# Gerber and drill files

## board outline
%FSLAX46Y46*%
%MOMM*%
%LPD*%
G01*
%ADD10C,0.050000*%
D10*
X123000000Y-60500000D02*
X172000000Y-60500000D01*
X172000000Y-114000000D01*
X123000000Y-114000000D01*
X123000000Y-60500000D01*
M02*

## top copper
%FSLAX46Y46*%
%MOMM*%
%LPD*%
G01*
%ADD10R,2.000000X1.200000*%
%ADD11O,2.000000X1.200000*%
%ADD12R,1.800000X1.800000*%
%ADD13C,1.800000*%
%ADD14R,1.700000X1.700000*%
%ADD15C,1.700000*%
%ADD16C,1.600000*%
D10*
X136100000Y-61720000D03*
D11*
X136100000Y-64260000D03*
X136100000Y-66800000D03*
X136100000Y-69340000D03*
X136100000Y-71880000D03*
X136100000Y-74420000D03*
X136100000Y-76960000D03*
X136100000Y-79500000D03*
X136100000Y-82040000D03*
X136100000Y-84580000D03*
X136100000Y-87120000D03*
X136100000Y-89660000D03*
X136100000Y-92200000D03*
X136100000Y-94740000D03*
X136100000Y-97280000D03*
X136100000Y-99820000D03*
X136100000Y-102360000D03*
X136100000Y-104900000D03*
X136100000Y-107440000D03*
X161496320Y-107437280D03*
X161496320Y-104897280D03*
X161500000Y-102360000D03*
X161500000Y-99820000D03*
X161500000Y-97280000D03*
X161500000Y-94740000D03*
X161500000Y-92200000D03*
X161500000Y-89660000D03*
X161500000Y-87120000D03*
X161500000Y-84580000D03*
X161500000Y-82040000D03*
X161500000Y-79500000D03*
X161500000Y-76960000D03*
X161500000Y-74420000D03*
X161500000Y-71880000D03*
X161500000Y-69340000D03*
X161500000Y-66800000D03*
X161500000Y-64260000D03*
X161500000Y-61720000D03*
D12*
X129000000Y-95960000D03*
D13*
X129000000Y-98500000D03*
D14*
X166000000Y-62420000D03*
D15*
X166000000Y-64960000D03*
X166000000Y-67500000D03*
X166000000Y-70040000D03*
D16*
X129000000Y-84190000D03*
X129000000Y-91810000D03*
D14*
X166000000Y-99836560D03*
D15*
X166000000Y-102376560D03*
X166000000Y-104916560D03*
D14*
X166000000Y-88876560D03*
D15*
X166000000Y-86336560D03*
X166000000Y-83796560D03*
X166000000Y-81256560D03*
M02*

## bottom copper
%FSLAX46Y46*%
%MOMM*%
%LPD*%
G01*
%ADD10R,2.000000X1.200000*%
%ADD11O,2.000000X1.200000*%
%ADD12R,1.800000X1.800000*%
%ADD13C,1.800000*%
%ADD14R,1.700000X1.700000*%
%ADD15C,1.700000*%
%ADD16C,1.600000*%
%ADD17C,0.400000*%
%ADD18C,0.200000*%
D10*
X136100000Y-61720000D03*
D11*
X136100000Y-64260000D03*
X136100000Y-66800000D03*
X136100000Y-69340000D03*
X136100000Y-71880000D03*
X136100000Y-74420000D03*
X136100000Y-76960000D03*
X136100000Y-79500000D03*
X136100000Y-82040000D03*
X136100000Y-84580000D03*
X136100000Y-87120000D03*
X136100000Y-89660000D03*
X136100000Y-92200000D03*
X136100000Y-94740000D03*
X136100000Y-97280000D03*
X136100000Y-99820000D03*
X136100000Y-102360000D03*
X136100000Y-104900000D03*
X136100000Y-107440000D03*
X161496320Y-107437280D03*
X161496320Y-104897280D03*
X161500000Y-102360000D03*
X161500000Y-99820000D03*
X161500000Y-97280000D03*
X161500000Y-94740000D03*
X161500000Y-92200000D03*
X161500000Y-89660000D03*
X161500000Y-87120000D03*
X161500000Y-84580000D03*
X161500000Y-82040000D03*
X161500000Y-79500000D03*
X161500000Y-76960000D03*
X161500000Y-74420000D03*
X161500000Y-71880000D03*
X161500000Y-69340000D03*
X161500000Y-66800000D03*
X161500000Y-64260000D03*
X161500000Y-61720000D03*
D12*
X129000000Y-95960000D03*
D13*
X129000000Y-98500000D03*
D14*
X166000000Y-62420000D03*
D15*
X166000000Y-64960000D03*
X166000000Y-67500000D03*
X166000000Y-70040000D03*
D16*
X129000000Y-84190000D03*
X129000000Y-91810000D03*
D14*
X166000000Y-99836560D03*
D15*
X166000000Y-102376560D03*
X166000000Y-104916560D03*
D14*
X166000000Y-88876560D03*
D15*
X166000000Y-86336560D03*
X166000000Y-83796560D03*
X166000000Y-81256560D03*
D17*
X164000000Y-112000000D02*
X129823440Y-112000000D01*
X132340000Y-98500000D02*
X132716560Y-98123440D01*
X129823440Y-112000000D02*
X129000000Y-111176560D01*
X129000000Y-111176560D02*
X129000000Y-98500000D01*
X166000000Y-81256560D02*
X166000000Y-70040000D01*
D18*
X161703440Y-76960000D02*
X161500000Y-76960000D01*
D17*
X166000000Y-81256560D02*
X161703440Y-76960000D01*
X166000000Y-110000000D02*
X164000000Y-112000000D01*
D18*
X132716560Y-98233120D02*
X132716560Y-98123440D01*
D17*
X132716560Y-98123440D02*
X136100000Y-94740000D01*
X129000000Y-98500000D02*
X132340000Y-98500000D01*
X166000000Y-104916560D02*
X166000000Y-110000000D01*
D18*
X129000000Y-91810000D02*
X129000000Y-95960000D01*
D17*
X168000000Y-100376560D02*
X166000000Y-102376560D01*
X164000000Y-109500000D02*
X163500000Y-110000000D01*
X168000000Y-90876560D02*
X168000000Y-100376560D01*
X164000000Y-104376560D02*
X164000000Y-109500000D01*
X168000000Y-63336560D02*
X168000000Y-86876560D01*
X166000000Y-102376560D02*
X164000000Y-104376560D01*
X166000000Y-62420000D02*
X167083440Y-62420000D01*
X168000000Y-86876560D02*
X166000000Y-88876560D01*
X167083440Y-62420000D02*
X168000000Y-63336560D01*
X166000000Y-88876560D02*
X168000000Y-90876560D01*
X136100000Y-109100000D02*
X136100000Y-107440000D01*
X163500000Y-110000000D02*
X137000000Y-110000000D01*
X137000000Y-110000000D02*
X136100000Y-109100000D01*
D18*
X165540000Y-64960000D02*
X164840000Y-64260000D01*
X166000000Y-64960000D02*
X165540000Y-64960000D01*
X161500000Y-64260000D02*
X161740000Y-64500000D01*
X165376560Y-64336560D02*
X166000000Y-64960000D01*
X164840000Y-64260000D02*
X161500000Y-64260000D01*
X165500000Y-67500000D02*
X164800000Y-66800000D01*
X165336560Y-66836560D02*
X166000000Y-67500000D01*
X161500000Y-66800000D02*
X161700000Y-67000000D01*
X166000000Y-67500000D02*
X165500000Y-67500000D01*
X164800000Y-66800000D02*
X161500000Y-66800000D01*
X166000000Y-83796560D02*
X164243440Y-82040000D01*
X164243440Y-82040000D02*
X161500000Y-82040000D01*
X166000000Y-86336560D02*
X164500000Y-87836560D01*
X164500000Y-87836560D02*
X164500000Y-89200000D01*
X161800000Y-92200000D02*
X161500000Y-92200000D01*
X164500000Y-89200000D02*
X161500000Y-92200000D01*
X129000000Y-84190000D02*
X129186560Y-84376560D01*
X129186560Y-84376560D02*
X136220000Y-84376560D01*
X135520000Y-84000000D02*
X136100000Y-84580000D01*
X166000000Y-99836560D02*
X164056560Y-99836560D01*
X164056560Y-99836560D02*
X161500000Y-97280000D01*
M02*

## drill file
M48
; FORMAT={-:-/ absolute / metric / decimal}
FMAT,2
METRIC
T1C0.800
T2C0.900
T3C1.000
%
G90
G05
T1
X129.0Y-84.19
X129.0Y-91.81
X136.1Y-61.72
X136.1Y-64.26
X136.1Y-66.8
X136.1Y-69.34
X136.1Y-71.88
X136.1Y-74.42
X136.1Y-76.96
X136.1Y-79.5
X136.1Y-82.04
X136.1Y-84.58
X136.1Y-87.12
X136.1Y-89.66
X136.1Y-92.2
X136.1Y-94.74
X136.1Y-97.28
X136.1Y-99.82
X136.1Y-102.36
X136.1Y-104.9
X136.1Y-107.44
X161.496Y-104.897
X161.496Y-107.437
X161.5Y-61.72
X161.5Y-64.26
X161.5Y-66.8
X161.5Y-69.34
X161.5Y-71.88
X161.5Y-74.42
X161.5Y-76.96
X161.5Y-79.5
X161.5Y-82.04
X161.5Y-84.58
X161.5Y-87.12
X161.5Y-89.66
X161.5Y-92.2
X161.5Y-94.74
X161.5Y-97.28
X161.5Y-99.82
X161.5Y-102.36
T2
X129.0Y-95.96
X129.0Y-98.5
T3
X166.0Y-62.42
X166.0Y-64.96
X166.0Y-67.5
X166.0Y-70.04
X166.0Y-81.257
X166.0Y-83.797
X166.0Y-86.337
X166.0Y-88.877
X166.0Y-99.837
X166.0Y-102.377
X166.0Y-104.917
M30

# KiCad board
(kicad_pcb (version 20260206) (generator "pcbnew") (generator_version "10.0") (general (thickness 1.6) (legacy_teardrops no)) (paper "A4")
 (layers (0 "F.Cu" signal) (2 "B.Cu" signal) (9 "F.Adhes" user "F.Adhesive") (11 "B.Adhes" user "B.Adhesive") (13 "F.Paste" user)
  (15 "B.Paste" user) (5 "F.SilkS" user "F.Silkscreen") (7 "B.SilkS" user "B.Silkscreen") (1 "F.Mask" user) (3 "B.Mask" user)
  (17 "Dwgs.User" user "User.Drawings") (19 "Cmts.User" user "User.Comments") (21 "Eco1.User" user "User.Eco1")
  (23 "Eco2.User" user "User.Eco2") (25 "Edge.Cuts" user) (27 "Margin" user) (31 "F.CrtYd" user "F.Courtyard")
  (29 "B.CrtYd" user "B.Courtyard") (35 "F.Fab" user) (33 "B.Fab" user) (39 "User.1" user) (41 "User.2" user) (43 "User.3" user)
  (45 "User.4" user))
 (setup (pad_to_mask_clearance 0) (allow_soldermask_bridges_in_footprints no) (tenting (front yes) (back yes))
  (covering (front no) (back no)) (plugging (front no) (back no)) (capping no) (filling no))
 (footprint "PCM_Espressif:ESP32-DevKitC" (layer "F.Cu") (at 136.1 61.72)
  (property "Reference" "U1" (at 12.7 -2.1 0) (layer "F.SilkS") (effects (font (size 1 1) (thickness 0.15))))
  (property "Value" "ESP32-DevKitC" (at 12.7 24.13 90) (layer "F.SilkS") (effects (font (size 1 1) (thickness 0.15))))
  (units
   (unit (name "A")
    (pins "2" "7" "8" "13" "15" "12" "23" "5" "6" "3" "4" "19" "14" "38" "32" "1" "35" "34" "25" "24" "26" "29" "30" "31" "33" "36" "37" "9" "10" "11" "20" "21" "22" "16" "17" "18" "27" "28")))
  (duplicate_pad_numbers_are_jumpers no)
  (pad "1" thru_hole rect (at 0 0 270) (size 1.2 2) (drill 0.8) (layers "*.Cu" "*.Mask") (remove_unused_layers no)
   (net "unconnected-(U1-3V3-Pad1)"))
  (pad "2" thru_hole oval (at 0 2.54 270) (size 1.2 2) (drill 0.8) (layers "*.Cu" "*.Mask") (remove_unused_layers no)
   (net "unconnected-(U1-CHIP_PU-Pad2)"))
  (pad "3" thru_hole oval (at 0 5.08 270) (size 1.2 2) (drill 0.8) (layers "*.Cu" "*.Mask") (remove_unused_layers no)
   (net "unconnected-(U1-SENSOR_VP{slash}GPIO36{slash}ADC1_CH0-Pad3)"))
  (pad "4" thru_hole oval (at 0 7.62 270) (size 1.2 2) (drill 0.8) (layers "*.Cu" "*.Mask") (remove_unused_layers no)
   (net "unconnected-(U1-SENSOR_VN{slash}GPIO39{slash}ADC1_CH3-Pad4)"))
  (pad "5" thru_hole oval (at 0 10.16 270) (size 1.2 2) (drill 0.8) (layers "*.Cu" "*.Mask") (remove_unused_layers no)
   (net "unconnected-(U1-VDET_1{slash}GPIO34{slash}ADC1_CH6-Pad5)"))
  (pad "6" thru_hole oval (at 0 12.7 270) (size 1.2 2) (drill 0.8) (layers "*.Cu" "*.Mask") (remove_unused_layers no)
   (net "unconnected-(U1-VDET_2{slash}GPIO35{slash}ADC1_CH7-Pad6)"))
  (pad "7" thru_hole oval (at 0 15.24 270) (size 1.2 2) (drill 0.8) (layers "*.Cu" "*.Mask") (remove_unused_layers no)
   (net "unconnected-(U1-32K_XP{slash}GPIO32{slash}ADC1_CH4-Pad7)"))
  (pad "8" thru_hole oval (at 0 17.78 270) (size 1.2 2) (drill 0.8) (layers "*.Cu" "*.Mask") (remove_unused_layers no)
   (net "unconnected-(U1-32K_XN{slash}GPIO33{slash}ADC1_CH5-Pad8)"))
  (pad "9" thru_hole oval (at 0 20.32 270) (size 1.2 2) (drill 0.8) (layers "*.Cu" "*.Mask") (remove_unused_layers no)
   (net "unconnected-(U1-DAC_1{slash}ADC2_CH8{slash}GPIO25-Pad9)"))
  (pad "10" thru_hole oval (at 0 22.86 270) (size 1.2 2) (drill 0.8) (layers "*.Cu" "*.Mask") (remove_unused_layers no)
   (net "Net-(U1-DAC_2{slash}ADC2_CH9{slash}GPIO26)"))
  (pad "11" thru_hole oval (at 0 25.4 270) (size 1.2 2) (drill 0.8) (layers "*.Cu" "*.Mask") (remove_unused_layers no)
   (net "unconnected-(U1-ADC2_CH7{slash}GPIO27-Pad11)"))
  (pad "12" thru_hole oval (at 0 27.94 270) (size 1.2 2) (drill 0.8) (layers "*.Cu" "*.Mask") (remove_unused_layers no)
   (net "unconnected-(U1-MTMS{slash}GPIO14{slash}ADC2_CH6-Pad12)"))
  (pad "13" thru_hole oval (at 0 30.48 270) (size 1.2 2) (drill 0.8) (layers "*.Cu" "*.Mask") (remove_unused_layers no)
   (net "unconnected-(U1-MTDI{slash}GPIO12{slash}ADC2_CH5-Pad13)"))
  (pad "14" thru_hole oval (at 0 33.02 270) (size 1.2 2) (drill 0.8) (layers "*.Cu" "*.Mask") (remove_unused_layers no) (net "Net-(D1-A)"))
  (pad "15" thru_hole oval (at 0 35.56 270) (size 1.2 2) (drill 0.8) (layers "*.Cu" "*.Mask") (remove_unused_layers no)
   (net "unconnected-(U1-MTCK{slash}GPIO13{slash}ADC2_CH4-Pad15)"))
  (pad "16" thru_hole oval (at 0 38.1 270) (size 1.2 2) (drill 0.8) (layers "*.Cu" "*.Mask") (remove_unused_layers no)
   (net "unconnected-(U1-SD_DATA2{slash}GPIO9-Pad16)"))
  (pad "17" thru_hole oval (at 0 40.64 270) (size 1.2 2) (drill 0.8) (layers "*.Cu" "*.Mask") (remove_unused_layers no)
   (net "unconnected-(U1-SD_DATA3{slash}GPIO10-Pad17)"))
  (pad "18" thru_hole oval (at 0 43.18 270) (size 1.2 2) (drill 0.8) (layers "*.Cu" "*.Mask") (remove_unused_layers no)
   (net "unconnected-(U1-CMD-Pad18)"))
  (pad "19" thru_hole oval (at 0 45.72 270) (size 1.2 2) (drill 0.8) (layers "*.Cu" "*.Mask") (remove_unused_layers no)
   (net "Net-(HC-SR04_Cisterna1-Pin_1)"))
  (pad "20" thru_hole oval (at 25.39632 45.71728 270) (size 1.2 2) (drill 0.8) (layers "*.Cu" "*.Mask") (remove_unused_layers no)
   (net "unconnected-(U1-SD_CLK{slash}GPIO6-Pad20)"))
  (pad "21" thru_hole oval (at 25.39632 43.17728 270) (size 1.2 2) (drill 0.8) (layers "*.Cu" "*.Mask") (remove_unused_layers no)
   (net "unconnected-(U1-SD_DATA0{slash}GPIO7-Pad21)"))
  (pad "22" thru_hole oval (at 25.4 40.64 270) (size 1.2 2) (drill 0.8) (layers "*.Cu" "*.Mask") (remove_unused_layers no)
   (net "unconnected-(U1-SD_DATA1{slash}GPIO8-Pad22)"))
  (pad "23" thru_hole oval (at 25.4 38.1 270) (size 1.2 2) (drill 0.8) (layers "*.Cu" "*.Mask") (remove_unused_layers no)
   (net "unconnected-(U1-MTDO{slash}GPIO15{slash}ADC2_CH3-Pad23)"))
  (pad "24" thru_hole oval (at 25.4 35.56 270) (size 1.2 2) (drill 0.8) (layers "*.Cu" "*.Mask") (remove_unused_layers no)
   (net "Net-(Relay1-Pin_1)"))
  (pad "25" thru_hole oval (at 25.4 33.02 270) (size 1.2 2) (drill 0.8) (layers "*.Cu" "*.Mask") (remove_unused_layers no)
   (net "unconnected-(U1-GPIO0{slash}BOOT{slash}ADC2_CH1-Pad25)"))
  (pad "26" thru_hole oval (at 25.4 30.48 270) (size 1.2 2) (drill 0.8) (layers "*.Cu" "*.Mask") (remove_unused_layers no)
   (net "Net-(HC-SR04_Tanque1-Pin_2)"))
  (pad "27" thru_hole oval (at 25.4 27.94 270) (size 1.2 2) (drill 0.8) (layers "*.Cu" "*.Mask") (remove_unused_layers no)
   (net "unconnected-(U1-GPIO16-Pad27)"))
  (pad "28" thru_hole oval (at 25.4 25.4 270) (size 1.2 2) (drill 0.8) (layers "*.Cu" "*.Mask") (remove_unused_layers no)
   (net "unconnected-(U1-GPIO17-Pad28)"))
  (pad "29" thru_hole oval (at 25.4 22.86 270) (size 1.2 2) (drill 0.8) (layers "*.Cu" "*.Mask") (remove_unused_layers no)
   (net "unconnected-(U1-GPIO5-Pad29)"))
  (pad "30" thru_hole oval (at 25.4 20.32 270) (size 1.2 2) (drill 0.8) (layers "*.Cu" "*.Mask") (remove_unused_layers no)
   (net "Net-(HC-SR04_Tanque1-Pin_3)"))
  (pad "31" thru_hole oval (at 25.4 17.78 270) (size 1.2 2) (drill 0.8) (layers "*.Cu" "*.Mask") (remove_unused_layers no)
   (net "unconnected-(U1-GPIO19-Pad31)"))
  (pad "32" thru_hole oval (at 25.4 15.24 270) (size 1.2 2) (drill 0.8) (layers "*.Cu" "*.Mask") (remove_unused_layers no)
   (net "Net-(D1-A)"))
  (pad "33" thru_hole oval (at 25.4 12.7 270) (size 1.2 2) (drill 0.8) (layers "*.Cu" "*.Mask") (remove_unused_layers no)
   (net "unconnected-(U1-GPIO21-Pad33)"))
  (pad "34" thru_hole oval (at 25.4 10.16 270) (size 1.2 2) (drill 0.8) (layers "*.Cu" "*.Mask") (remove_unused_layers no)
   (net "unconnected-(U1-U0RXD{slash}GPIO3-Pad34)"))
  (pad "35" thru_hole oval (at 25.4 7.62 270) (size 1.2 2) (drill 0.8) (layers "*.Cu" "*.Mask") (remove_unused_layers no)
   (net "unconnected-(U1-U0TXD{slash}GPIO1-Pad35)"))
  (pad "36" thru_hole oval (at 25.4 5.08 270) (size 1.2 2) (drill 0.8) (layers "*.Cu" "*.Mask") (remove_unused_layers no)
   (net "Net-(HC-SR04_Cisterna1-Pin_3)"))
  (pad "37" thru_hole oval (at 25.4 2.54 270) (size 1.2 2) (drill 0.8) (layers "*.Cu" "*.Mask") (remove_unused_layers no)
   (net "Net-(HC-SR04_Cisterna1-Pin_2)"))
  (pad "38" thru_hole oval (at 25.4 0 270) (size 1.2 2) (drill 0.8) (layers "*.Cu" "*.Mask") (remove_unused_layers no) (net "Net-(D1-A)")))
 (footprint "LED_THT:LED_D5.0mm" (layer "F.Cu") (at 129 95.96 -90)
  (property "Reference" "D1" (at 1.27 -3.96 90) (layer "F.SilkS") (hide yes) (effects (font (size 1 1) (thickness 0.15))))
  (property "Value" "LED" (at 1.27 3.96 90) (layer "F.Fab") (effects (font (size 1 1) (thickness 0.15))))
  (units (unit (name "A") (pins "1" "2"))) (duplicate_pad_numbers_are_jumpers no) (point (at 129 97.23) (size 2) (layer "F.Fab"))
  (pad "1" thru_hole rect (at 0 0 270) (size 1.8 1.8) (drill 0.9) (layers "*.Cu" "*.Mask") (remove_unused_layers no) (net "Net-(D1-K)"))
  (pad "2" thru_hole circle (at 2.54 0 270) (size 1.8 1.8) (drill 0.9) (layers "*.Cu" "*.Mask") (remove_unused_layers no) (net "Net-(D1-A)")))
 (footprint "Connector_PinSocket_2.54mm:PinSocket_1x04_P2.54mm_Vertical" (layer "F.Cu") (at 166 62.42)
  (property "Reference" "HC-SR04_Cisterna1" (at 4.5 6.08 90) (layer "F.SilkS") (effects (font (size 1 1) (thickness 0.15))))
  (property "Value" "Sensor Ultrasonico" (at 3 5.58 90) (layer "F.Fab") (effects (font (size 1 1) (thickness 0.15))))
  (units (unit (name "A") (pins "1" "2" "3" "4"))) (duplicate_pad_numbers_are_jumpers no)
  (pad "1" thru_hole rect (at 0 0) (size 1.7 1.7) (drill 1) (layers "*.Cu" "*.Mask") (remove_unused_layers no)
   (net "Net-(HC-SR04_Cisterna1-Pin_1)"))
  (pad "2" thru_hole circle (at 0 2.54) (size 1.7 1.7) (drill 1) (layers "*.Cu" "*.Mask") (remove_unused_layers no)
   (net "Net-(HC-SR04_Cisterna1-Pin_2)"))
  (pad "3" thru_hole circle (at 0 5.08) (size 1.7 1.7) (drill 1) (layers "*.Cu" "*.Mask") (remove_unused_layers no)
   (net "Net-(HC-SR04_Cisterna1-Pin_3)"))
  (pad "4" thru_hole circle (at 0 7.62) (size 1.7 1.7) (drill 1) (layers "*.Cu" "*.Mask") (remove_unused_layers no) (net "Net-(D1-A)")))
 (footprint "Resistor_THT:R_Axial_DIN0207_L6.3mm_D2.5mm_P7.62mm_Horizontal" (layer "F.Cu") (at 129 84.19 -90)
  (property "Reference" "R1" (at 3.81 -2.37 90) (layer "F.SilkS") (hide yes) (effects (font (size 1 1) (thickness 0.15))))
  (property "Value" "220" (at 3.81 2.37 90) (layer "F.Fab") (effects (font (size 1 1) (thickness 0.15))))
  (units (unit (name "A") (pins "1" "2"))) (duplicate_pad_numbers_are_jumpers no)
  (pad "1" thru_hole circle (at 0 0 270) (size 1.6 1.6) (drill 0.8) (layers "*.Cu" "*.Mask") (remove_unused_layers no)
   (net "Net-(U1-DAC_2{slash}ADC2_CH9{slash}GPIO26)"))
  (pad "2" thru_hole circle (at 7.62 0 270) (size 1.6 1.6) (drill 0.8) (layers "*.Cu" "*.Mask") (remove_unused_layers no) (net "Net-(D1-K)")))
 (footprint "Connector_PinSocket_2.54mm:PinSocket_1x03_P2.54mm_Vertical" (layer "F.Cu") (at 166 99.83656)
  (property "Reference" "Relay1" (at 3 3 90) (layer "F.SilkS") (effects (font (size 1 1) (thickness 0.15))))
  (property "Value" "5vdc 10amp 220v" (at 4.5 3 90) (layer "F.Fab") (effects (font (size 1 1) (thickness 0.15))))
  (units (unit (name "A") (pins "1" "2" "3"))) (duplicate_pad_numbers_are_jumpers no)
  (pad "1" thru_hole rect (at 0 0) (size 1.7 1.7) (drill 1) (layers "*.Cu" "*.Mask") (remove_unused_layers no) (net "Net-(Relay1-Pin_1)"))
  (pad "2" thru_hole circle (at 0 2.54) (size 1.7 1.7) (drill 1) (layers "*.Cu" "*.Mask") (remove_unused_layers no)
   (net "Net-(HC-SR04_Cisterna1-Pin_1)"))
  (pad "3" thru_hole circle (at 0 5.08) (size 1.7 1.7) (drill 1) (layers "*.Cu" "*.Mask") (remove_unused_layers no) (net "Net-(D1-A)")))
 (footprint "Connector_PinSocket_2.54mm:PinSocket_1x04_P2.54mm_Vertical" (layer "F.Cu") (at 166 88.87656 180)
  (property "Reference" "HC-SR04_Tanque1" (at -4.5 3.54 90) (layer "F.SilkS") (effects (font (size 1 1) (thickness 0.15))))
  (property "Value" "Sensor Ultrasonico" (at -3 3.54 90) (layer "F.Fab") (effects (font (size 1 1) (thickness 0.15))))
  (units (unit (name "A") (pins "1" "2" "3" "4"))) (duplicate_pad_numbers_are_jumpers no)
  (pad "1" thru_hole rect (at 0 0 180) (size 1.7 1.7) (drill 1) (layers "*.Cu" "*.Mask") (remove_unused_layers no)
   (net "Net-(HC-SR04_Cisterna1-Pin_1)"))
  (pad "2" thru_hole circle (at 0 2.54 180) (size 1.7 1.7) (drill 1) (layers "*.Cu" "*.Mask") (remove_unused_layers no)
   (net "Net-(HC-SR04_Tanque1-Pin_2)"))
  (pad "3" thru_hole circle (at 0 5.08 180) (size 1.7 1.7) (drill 1) (layers "*.Cu" "*.Mask") (remove_unused_layers no)
   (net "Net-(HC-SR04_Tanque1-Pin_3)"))
  (pad "4" thru_hole circle (at 0 7.62 180) (size 1.7 1.7) (drill 1) (layers "*.Cu" "*.Mask") (remove_unused_layers no) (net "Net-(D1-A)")))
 (gr_rect (start 123 60.5) (end 172 114) (stroke (width 0.05) (type default)) (fill no) (layer "Edge.Cuts"))
 (segment (start 164 112) (end 129.82344 112) (width 0.4) (layer "B.Cu") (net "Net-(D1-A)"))
 (segment (start 132.34 98.5) (end 132.71656 98.12344) (width 0.4) (layer "B.Cu") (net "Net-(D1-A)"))
 (segment (start 129.82344 112) (end 129 111.17656) (width 0.4) (layer "B.Cu") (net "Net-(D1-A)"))
 (segment (start 129 111.17656) (end 129 98.5) (width 0.4) (layer "B.Cu") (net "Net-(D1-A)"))
 (segment (start 166 81.25656) (end 166 70.04) (width 0.4) (layer "B.Cu") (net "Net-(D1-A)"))
 (segment (start 161.70344 76.96) (end 161.5 76.96) (width 0.2) (layer "B.Cu") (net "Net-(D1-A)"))
 (segment (start 166 81.25656) (end 161.70344 76.96) (width 0.4) (layer "B.Cu") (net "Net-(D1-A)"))
 (segment (start 166 110) (end 164 112) (width 0.4) (layer "B.Cu") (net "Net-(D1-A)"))
 (segment (start 132.71656 98.23312) (end 132.71656 98.12344) (width 0.2) (layer "B.Cu") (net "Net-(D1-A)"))
 (segment (start 132.71656 98.12344) (end 136.1 94.74) (width 0.4) (layer "B.Cu") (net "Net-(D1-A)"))
 (segment (start 129 98.5) (end 132.34 98.5) (width 0.4) (layer "B.Cu") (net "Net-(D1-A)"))
 (segment (start 166 104.91656) (end 166 110) (width 0.4) (layer "B.Cu") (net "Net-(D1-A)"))
 (segment (start 129 91.81) (end 129 95.96) (width 0.2) (layer "B.Cu") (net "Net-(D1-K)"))
 (segment (start 168 100.37656) (end 166 102.37656) (width 0.4) (layer "B.Cu") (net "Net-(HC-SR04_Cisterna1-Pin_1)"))
 (segment (start 164 109.5) (end 163.5 110) (width 0.4) (layer "B.Cu") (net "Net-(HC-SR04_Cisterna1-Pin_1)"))
 (segment (start 168 90.87656) (end 168 100.37656) (width 0.4) (layer "B.Cu") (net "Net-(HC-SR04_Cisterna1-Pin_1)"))
 (segment (start 164 104.37656) (end 164 109.5) (width 0.4) (layer "B.Cu") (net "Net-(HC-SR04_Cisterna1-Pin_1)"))
 (segment (start 168 63.33656) (end 168 86.87656) (width 0.4) (layer "B.Cu") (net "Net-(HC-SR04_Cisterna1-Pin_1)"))
 (segment (start 166 102.37656) (end 164 104.37656) (width 0.4) (layer "B.Cu") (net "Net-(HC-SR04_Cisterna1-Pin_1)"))
 (segment (start 166 62.42) (end 167.08344 62.42) (width 0.4) (layer "B.Cu") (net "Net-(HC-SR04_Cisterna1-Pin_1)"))
 (segment (start 168 86.87656) (end 166 88.87656) (width 0.4) (layer "B.Cu") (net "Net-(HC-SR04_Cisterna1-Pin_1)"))
 (segment (start 167.08344 62.42) (end 168 63.33656) (width 0.4) (layer "B.Cu") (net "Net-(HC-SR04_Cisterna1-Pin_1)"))
 (segment (start 166 88.87656) (end 168 90.87656) (width 0.4) (layer "B.Cu") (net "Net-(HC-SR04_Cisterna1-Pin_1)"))
 (segment (start 136.1 109.1) (end 136.1 107.44) (width 0.4) (layer "B.Cu") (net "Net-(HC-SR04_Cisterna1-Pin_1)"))
 (segment (start 163.5 110) (end 137 110) (width 0.4) (layer "B.Cu") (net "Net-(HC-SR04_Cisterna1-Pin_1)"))
 (segment (start 137 110) (end 136.1 109.1) (width 0.4) (layer "B.Cu") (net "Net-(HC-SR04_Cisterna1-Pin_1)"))
 (segment (start 165.54 64.96) (end 164.84 64.26) (width 0.2) (layer "B.Cu") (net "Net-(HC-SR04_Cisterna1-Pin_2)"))
 (segment (start 166 64.96) (end 165.54 64.96) (width 0.2) (layer "B.Cu") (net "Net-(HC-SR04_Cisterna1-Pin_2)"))
 (segment (start 161.5 64.26) (end 161.74 64.5) (width 0.2) (layer "B.Cu") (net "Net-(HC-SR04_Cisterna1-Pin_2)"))
 (segment (start 165.37656 64.33656) (end 166 64.96) (width 0.2) (layer "B.Cu") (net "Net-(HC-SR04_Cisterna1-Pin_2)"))
 (segment (start 164.84 64.26) (end 161.5 64.26) (width 0.2) (layer "B.Cu") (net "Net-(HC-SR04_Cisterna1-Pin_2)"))
 (segment (start 165.5 67.5) (end 164.8 66.8) (width 0.2) (layer "B.Cu") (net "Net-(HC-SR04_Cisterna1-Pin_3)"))
 (segment (start 165.33656 66.83656) (end 166 67.5) (width 0.2) (layer "B.Cu") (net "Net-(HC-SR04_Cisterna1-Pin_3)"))
 (segment (start 161.5 66.8) (end 161.7 67) (width 0.2) (layer "B.Cu") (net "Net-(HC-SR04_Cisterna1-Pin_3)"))
 (segment (start 166 67.5) (end 165.5 67.5) (width 0.2) (layer "B.Cu") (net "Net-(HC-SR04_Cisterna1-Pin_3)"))
 (segment (start 164.8 66.8) (end 161.5 66.8) (width 0.2) (layer "B.Cu") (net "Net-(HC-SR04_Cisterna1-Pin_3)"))
 (segment (start 166 83.79656) (end 164.24344 82.04) (width 0.2) (layer "B.Cu") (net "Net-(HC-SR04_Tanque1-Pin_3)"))
 (segment (start 164.24344 82.04) (end 161.5 82.04) (width 0.2) (layer "B.Cu") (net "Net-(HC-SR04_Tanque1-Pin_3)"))
 (segment (start 166 86.33656) (end 164.5 87.83656) (width 0.2) (layer "B.Cu") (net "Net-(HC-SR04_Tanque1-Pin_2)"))
 (segment (start 164.5 87.83656) (end 164.5 89.2) (width 0.2) (layer "B.Cu") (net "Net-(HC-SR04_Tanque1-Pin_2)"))
 (segment (start 161.8 92.2) (end 161.5 92.2) (width 0.2) (layer "B.Cu") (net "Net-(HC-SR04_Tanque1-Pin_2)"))
 (segment (start 164.5 89.2) (end 161.5 92.2) (width 0.2) (layer "B.Cu") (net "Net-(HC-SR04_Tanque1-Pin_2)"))
 (segment (start 129 84.19) (end 129.18656 84.37656) (width 0.2) (layer "B.Cu") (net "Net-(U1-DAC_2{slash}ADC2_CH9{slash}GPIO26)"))
 (segment (start 129.18656 84.37656) (end 136.22 84.37656) (width 0.2) (layer "B.Cu") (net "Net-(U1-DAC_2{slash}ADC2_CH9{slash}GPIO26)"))
 (segment (start 135.52 84) (end 136.1 84.58) (width 0.2) (layer "B.Cu") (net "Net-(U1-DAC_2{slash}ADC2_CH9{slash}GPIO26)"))
 (segment (start 166 99.83656) (end 164.05656 99.83656) (width 0.2) (layer "B.Cu") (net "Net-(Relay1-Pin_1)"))
 (segment (start 164.05656 99.83656) (end 161.5 97.28) (width 0.2) (layer "B.Cu") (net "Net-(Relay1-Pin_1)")))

